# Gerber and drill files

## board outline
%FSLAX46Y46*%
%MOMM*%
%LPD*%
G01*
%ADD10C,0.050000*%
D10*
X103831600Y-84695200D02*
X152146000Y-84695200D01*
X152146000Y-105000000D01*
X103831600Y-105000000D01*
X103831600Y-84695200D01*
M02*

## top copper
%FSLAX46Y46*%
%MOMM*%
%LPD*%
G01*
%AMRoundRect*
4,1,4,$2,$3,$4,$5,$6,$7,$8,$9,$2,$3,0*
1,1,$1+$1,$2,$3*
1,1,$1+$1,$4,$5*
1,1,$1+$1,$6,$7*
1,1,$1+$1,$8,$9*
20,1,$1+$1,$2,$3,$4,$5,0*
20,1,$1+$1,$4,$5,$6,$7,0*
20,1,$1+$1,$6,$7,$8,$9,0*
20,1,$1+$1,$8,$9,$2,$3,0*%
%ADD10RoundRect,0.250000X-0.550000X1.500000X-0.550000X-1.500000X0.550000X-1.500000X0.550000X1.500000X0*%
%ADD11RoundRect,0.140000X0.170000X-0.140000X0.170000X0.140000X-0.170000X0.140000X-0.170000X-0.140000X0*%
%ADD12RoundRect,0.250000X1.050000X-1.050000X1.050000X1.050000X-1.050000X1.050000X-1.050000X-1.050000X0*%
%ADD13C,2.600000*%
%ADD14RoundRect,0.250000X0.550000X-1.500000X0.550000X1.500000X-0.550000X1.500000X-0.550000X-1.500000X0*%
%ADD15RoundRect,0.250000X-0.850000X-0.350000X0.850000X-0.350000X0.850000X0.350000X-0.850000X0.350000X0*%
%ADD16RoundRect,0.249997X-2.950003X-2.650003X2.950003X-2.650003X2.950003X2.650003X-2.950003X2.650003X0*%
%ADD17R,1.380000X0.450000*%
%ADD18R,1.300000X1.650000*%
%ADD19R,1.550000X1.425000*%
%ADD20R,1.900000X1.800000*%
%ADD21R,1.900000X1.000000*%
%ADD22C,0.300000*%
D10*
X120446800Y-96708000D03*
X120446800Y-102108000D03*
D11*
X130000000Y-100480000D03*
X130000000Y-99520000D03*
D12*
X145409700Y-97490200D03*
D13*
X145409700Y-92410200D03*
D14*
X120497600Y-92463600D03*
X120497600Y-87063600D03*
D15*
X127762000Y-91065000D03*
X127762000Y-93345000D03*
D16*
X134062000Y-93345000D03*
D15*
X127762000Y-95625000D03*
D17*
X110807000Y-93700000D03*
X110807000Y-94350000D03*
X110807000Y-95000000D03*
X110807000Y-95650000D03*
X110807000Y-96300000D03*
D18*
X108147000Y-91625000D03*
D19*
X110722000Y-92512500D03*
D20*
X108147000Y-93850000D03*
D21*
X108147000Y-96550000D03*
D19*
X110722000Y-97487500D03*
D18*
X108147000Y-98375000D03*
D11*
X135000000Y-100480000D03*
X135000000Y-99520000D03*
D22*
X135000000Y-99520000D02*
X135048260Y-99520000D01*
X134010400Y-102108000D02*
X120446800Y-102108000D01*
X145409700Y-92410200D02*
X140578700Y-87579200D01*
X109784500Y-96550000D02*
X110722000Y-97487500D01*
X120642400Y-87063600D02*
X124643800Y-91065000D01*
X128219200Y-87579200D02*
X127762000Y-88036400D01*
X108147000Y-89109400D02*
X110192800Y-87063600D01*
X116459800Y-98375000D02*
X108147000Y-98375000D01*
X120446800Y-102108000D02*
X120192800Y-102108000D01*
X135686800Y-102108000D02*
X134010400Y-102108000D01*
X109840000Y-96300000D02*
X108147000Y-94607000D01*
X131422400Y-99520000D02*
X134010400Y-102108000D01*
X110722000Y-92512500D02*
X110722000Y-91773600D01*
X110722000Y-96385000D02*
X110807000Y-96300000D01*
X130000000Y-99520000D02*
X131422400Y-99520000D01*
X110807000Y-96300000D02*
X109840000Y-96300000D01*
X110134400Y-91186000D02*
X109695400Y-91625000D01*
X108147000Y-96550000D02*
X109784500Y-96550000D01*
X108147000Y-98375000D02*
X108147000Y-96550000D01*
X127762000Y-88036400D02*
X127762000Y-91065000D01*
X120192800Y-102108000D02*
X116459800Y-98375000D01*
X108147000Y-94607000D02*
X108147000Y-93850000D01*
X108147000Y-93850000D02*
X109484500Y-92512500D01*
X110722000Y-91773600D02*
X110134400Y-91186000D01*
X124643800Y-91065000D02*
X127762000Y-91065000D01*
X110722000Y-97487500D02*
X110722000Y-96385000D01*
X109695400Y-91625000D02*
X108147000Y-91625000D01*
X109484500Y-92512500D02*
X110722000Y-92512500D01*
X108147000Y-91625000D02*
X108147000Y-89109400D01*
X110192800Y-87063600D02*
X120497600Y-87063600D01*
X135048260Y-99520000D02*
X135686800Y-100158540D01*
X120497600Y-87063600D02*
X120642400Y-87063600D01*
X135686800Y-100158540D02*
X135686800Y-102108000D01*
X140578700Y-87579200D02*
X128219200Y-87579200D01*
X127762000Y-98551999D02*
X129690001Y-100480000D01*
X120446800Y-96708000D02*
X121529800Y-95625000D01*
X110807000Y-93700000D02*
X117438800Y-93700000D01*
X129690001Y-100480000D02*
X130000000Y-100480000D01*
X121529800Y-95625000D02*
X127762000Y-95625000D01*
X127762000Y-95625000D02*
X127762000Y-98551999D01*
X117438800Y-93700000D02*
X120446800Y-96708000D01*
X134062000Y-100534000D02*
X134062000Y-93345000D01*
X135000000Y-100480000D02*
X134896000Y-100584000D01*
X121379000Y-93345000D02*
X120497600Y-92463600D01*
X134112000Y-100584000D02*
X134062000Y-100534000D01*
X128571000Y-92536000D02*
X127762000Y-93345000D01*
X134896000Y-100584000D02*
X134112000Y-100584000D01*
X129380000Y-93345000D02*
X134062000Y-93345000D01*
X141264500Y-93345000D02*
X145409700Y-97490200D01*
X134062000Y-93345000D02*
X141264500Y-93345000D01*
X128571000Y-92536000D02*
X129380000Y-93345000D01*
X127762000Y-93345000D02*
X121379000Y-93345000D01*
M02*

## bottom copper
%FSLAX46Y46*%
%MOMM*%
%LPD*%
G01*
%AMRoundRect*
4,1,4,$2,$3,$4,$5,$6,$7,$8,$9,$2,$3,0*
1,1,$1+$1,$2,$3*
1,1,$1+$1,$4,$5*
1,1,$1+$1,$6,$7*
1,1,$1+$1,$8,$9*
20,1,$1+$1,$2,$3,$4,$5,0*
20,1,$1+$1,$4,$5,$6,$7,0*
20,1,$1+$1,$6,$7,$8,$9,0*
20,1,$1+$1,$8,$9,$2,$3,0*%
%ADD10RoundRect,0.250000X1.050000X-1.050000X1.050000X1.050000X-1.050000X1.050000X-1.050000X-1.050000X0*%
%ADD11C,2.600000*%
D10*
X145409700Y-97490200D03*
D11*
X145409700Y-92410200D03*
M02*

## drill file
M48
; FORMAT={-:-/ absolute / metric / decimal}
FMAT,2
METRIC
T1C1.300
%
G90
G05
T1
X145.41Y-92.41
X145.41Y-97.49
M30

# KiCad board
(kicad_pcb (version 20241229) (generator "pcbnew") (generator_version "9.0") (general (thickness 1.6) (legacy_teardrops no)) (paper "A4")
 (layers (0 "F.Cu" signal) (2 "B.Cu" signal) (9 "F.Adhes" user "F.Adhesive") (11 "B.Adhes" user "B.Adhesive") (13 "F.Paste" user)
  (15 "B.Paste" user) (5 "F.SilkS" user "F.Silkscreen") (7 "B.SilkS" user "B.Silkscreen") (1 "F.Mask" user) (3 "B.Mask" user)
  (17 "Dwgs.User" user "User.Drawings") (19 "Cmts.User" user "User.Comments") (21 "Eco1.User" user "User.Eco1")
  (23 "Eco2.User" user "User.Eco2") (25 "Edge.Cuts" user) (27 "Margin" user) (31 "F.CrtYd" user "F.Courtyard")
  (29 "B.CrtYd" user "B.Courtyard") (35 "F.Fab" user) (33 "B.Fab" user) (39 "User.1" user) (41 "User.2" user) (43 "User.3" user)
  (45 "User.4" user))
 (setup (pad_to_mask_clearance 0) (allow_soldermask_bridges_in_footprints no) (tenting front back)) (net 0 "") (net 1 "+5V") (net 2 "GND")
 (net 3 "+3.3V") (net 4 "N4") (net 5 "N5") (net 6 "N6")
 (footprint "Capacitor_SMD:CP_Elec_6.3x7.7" (layer "F.Cu") (at 120.4468 99.408 -90)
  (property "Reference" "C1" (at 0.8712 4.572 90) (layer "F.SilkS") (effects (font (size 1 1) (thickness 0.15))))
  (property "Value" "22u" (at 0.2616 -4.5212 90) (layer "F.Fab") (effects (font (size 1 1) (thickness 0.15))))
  (pad "1" smd roundrect (at -2.7 0 270) (size 3.5 1.6) (layers "F.Cu" "F.Mask" "F.Paste") (roundrect_rratio 0.15625) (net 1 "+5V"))
  (pad "2" smd roundrect (at 2.7 0 270) (size 3.5 1.6) (layers "F.Cu" "F.Mask" "F.Paste") (roundrect_rratio 0.15625) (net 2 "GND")))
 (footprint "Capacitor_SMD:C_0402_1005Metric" (layer "F.Cu") (at 130 100 90)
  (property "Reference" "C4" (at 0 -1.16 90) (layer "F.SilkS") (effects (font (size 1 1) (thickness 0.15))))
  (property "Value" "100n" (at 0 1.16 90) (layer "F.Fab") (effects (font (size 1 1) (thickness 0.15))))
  (pad "1" smd roundrect (at -0.48 0 90) (size 0.56 0.62) (layers "F.Cu" "F.Mask" "F.Paste") (roundrect_rratio 0.25) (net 1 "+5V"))
  (pad "2" smd roundrect (at 0.48 0 90) (size 0.56 0.62) (layers "F.Cu" "F.Mask" "F.Paste") (roundrect_rratio 0.25) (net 2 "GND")))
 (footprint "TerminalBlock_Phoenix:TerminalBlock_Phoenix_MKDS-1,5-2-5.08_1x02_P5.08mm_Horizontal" (layer "F.Cu") (at 145.4097 97.4902 90)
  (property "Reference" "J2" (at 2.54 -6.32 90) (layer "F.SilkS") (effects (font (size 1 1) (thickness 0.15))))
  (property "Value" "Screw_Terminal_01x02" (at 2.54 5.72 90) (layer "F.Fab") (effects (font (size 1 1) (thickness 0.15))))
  (pad "1" thru_hole roundrect (at 0 0 90) (size 2.6 2.6) (drill 1.3) (layers "*.Cu" "*.Mask") (remove_unused_layers no)
   (roundrect_rratio 0.096154) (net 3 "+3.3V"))
  (pad "2" thru_hole circle (at 5.08 0 90) (size 2.6 2.6) (drill 1.3) (layers "*.Cu" "*.Mask") (remove_unused_layers no) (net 2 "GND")))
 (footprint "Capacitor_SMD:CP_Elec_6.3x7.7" (layer "F.Cu") (at 120.4976 89.7636 90)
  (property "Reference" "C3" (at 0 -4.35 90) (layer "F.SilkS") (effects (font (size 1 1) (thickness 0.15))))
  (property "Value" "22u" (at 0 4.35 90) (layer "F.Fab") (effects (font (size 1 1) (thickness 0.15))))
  (pad "1" smd roundrect (at -2.7 0 90) (size 3.5 1.6) (layers "F.Cu" "F.Mask" "F.Paste") (roundrect_rratio 0.15625) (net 3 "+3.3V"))
  (pad "2" smd roundrect (at 2.7 0 90) (size 3.5 1.6) (layers "F.Cu" "F.Mask" "F.Paste") (roundrect_rratio 0.15625) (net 2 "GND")))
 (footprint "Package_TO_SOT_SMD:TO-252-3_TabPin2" (layer "F.Cu") (at 132.802 93.345)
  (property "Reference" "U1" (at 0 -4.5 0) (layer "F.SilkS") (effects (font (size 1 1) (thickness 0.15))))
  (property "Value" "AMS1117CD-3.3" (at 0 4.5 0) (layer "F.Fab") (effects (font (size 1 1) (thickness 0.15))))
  (pad "" smd roundrect (at -0.415 -1.525) (size 3.05 2.75) (layers "F.Paste") (roundrect_rratio 0.090909))
  (pad "" smd roundrect (at -0.415 1.525) (size 3.05 2.75) (layers "F.Paste") (roundrect_rratio 0.090909))
  (pad "" smd roundrect (at 2.935 -1.525) (size 3.05 2.75) (layers "F.Paste") (roundrect_rratio 0.090909))
  (pad "" smd roundrect (at 2.935 1.525) (size 3.05 2.75) (layers "F.Paste") (roundrect_rratio 0.090909))
  (pad "1" smd roundrect (at -5.04 -2.28) (size 2.2 1.2) (layers "F.Cu" "F.Mask" "F.Paste") (roundrect_rratio 0.208333) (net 2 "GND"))
  (pad "2" smd roundrect (at -5.04 0) (size 2.2 1.2) (layers "F.Cu" "F.Mask" "F.Paste") (roundrect_rratio 0.208333) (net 3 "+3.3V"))
  (pad "2" smd roundrect (at 1.26 0) (size 6.4 5.8) (layers "F.Cu" "F.Mask") (roundrect_rratio 0.043103) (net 3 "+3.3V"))
  (pad "3" smd roundrect (at -5.04 2.28) (size 2.2 1.2) (layers "F.Cu" "F.Mask" "F.Paste") (roundrect_rratio 0.208333) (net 1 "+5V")))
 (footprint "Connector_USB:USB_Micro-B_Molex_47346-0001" (layer "F.Cu") (at 109.347 95 -90)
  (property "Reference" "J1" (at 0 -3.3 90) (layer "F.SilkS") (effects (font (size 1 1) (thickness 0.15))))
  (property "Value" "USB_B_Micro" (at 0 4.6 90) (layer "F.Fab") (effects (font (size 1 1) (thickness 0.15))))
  (pad "1" smd rect (at -1.3 -1.46 270) (size 0.45 1.38) (layers "F.Cu" "F.Mask" "F.Paste") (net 1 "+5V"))
  (pad "2" smd rect (at -0.65 -1.46 270) (size 0.45 1.38) (layers "F.Cu" "F.Mask" "F.Paste") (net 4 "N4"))
  (pad "3" smd rect (at 0 -1.46 270) (size 0.45 1.38) (layers "F.Cu" "F.Mask" "F.Paste") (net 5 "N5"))
  (pad "4" smd rect (at 0.65 -1.46 270) (size 0.45 1.38) (layers "F.Cu" "F.Mask" "F.Paste") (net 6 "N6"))
  (pad "5" smd rect (at 1.3 -1.46 270) (size 0.45 1.38) (layers "F.Cu" "F.Mask" "F.Paste") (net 2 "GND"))
  (pad "6" smd rect (at -3.375 1.2 270) (size 1.65 1.3) (layers "F.Cu" "F.Mask" "F.Paste") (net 2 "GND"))
  (pad "6" smd rect (at -2.4875 -1.375 270) (size 1.425 1.55) (layers "F.Cu" "F.Mask" "F.Paste") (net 2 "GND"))
  (pad "6" smd rect (at -1.15 1.2 270) (size 1.8 1.9) (layers "F.Cu" "F.Mask" "F.Paste") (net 2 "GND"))
  (pad "6" smd rect (at 1.55 1.2 270) (size 1 1.9) (layers "F.Cu" "F.Mask" "F.Paste") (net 2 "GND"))
  (pad "6" smd rect (at 2.4875 -1.375 270) (size 1.425 1.55) (layers "F.Cu" "F.Mask" "F.Paste") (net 2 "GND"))
  (pad "6" smd rect (at 3.375 1.2 270) (size 1.65 1.3) (layers "F.Cu" "F.Mask" "F.Paste") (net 2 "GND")))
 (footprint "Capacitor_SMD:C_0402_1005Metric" (layer "F.Cu") (at 135 100 90)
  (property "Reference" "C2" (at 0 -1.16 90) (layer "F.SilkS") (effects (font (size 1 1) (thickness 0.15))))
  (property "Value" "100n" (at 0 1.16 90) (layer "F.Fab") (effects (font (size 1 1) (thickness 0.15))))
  (pad "1" smd roundrect (at -0.48 0 90) (size 0.56 0.62) (layers "F.Cu" "F.Mask" "F.Paste") (roundrect_rratio 0.25) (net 3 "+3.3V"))
  (pad "2" smd roundrect (at 0.48 0 90) (size 0.56 0.62) (layers "F.Cu" "F.Mask" "F.Paste") (roundrect_rratio 0.25) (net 2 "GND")))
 (gr_rect (start 103.8316 84.6952) (end 152.146 105) (stroke (width 0.05) (type default)) (fill no) (layer "Edge.Cuts"))
 (segment (start 135 99.52) (end 135.04826 99.52) (width 0.3) (layer "F.Cu") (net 2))
 (segment (start 134.0104 102.108) (end 120.4468 102.108) (width 0.3) (layer "F.Cu") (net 2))
 (segment (start 145.4097 92.4102) (end 140.5787 87.5792) (width 0.3) (layer "F.Cu") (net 2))
 (segment (start 109.7845 96.55) (end 110.722 97.4875) (width 0.3) (layer "F.Cu") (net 2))
 (segment (start 120.6424 87.0636) (end 124.6438 91.065) (width 0.3) (layer "F.Cu") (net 2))
 (segment (start 128.2192 87.5792) (end 127.762 88.0364) (width 0.3) (layer "F.Cu") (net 2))
 (segment (start 108.147 89.1094) (end 110.1928 87.0636) (width 0.3) (layer "F.Cu") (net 2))
 (segment (start 116.4598 98.375) (end 108.147 98.375) (width 0.3) (layer "F.Cu") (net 2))
 (segment (start 120.4468 102.108) (end 120.1928 102.108) (width 0.3) (layer "F.Cu") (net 2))
 (segment (start 135.6868 102.108) (end 134.0104 102.108) (width 0.3) (layer "F.Cu") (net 2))
 (segment (start 109.84 96.3) (end 108.147 94.607) (width 0.3) (layer "F.Cu") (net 2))
 (segment (start 131.4224 99.52) (end 134.0104 102.108) (width 0.3) (layer "F.Cu") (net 2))
 (segment (start 110.722 92.5125) (end 110.722 91.7736) (width 0.3) (layer "F.Cu") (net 2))
 (segment (start 110.722 96.385) (end 110.807 96.3) (width 0.3) (layer "F.Cu") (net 2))
 (segment (start 130 99.52) (end 131.4224 99.52) (width 0.3) (layer "F.Cu") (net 2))
 (segment (start 110.807 96.3) (end 109.84 96.3) (width 0.3) (layer "F.Cu") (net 2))
 (segment (start 110.1344 91.186) (end 109.6954 91.625) (width 0.3) (layer "F.Cu") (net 2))
 (segment (start 108.147 96.55) (end 109.7845 96.55) (width 0.3) (layer "F.Cu") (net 2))
 (segment (start 108.147 98.375) (end 108.147 96.55) (width 0.3) (layer "F.Cu") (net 2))
 (segment (start 127.762 88.0364) (end 127.762 91.065) (width 0.3) (layer "F.Cu") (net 2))
 (segment (start 120.1928 102.108) (end 116.4598 98.375) (width 0.3) (layer "F.Cu") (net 2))
 (segment (start 108.147 94.607) (end 108.147 93.85) (width 0.3) (layer "F.Cu") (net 2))
 (segment (start 108.147 93.85) (end 109.4845 92.5125) (width 0.3) (layer "F.Cu") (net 2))
 (segment (start 110.722 91.7736) (end 110.1344 91.186) (width 0.3) (layer "F.Cu") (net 2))
 (segment (start 124.6438 91.065) (end 127.762 91.065) (width 0.3) (layer "F.Cu") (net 2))
 (segment (start 110.722 97.4875) (end 110.722 96.385) (width 0.3) (layer "F.Cu") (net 2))
 (segment (start 109.6954 91.625) (end 108.147 91.625) (width 0.3) (layer "F.Cu") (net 2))
 (segment (start 109.4845 92.5125) (end 110.722 92.5125) (width 0.3) (layer "F.Cu") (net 2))
 (segment (start 108.147 91.625) (end 108.147 89.1094) (width 0.3) (layer "F.Cu") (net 2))
 (segment (start 110.1928 87.0636) (end 120.4976 87.0636) (width 0.3) (layer "F.Cu") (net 2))
 (segment (start 135.04826 99.52) (end 135.6868 100.15854) (width 0.3) (layer "F.Cu") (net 2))
 (segment (start 120.4976 87.0636) (end 120.6424 87.0636) (width 0.3) (layer "F.Cu") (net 2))
 (segment (start 135.6868 100.15854) (end 135.6868 102.108) (width 0.3) (layer "F.Cu") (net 2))
 (segment (start 140.5787 87.5792) (end 128.2192 87.5792) (width 0.3) (layer "F.Cu") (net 2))
 (segment (start 127.762 98.551999) (end 129.690001 100.48) (width 0.3) (layer "F.Cu") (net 1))
 (segment (start 120.4468 96.708) (end 121.5298 95.625) (width 0.3) (layer "F.Cu") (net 1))
 (segment (start 110.807 93.7) (end 117.4388 93.7) (width 0.3) (layer "F.Cu") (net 1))
 (segment (start 129.690001 100.48) (end 130 100.48) (width 0.3) (layer "F.Cu") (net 1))
 (segment (start 121.5298 95.625) (end 127.762 95.625) (width 0.3) (layer "F.Cu") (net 1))
 (segment (start 127.762 95.625) (end 127.762 98.551999) (width 0.3) (layer "F.Cu") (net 1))
 (segment (start 117.4388 93.7) (end 120.4468 96.708) (width 0.3) (layer "F.Cu") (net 1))
 (segment (start 134.062 100.534) (end 134.062 93.345) (width 0.3) (layer "F.Cu") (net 3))
 (segment (start 135 100.48) (end 134.896 100.584) (width 0.3) (layer "F.Cu") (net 3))
 (segment (start 121.379 93.345) (end 120.4976 92.4636) (width 0.3) (layer "F.Cu") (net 3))
 (segment (start 134.112 100.584) (end 134.062 100.534) (width 0.3) (layer "F.Cu") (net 3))
 (segment (start 128.571 92.536) (end 127.762 93.345) (width 0.3) (layer "F.Cu") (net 3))
 (segment (start 134.896 100.584) (end 134.112 100.584) (width 0.3) (layer "F.Cu") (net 3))
 (segment (start 129.38 93.345) (end 134.062 93.345) (width 0.3) (layer "F.Cu") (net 3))
 (segment (start 141.2645 93.345) (end 145.4097 97.4902) (width 0.3) (layer "F.Cu") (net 3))
 (segment (start 134.062 93.345) (end 141.2645 93.345) (width 0.3) (layer "F.Cu") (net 3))
 (segment (start 128.571 92.536) (end 129.38 93.345) (width 0.3) (layer "F.Cu") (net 3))
 (segment (start 127.762 93.345) (end 121.379 93.345) (width 0.3) (layer "F.Cu") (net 3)))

